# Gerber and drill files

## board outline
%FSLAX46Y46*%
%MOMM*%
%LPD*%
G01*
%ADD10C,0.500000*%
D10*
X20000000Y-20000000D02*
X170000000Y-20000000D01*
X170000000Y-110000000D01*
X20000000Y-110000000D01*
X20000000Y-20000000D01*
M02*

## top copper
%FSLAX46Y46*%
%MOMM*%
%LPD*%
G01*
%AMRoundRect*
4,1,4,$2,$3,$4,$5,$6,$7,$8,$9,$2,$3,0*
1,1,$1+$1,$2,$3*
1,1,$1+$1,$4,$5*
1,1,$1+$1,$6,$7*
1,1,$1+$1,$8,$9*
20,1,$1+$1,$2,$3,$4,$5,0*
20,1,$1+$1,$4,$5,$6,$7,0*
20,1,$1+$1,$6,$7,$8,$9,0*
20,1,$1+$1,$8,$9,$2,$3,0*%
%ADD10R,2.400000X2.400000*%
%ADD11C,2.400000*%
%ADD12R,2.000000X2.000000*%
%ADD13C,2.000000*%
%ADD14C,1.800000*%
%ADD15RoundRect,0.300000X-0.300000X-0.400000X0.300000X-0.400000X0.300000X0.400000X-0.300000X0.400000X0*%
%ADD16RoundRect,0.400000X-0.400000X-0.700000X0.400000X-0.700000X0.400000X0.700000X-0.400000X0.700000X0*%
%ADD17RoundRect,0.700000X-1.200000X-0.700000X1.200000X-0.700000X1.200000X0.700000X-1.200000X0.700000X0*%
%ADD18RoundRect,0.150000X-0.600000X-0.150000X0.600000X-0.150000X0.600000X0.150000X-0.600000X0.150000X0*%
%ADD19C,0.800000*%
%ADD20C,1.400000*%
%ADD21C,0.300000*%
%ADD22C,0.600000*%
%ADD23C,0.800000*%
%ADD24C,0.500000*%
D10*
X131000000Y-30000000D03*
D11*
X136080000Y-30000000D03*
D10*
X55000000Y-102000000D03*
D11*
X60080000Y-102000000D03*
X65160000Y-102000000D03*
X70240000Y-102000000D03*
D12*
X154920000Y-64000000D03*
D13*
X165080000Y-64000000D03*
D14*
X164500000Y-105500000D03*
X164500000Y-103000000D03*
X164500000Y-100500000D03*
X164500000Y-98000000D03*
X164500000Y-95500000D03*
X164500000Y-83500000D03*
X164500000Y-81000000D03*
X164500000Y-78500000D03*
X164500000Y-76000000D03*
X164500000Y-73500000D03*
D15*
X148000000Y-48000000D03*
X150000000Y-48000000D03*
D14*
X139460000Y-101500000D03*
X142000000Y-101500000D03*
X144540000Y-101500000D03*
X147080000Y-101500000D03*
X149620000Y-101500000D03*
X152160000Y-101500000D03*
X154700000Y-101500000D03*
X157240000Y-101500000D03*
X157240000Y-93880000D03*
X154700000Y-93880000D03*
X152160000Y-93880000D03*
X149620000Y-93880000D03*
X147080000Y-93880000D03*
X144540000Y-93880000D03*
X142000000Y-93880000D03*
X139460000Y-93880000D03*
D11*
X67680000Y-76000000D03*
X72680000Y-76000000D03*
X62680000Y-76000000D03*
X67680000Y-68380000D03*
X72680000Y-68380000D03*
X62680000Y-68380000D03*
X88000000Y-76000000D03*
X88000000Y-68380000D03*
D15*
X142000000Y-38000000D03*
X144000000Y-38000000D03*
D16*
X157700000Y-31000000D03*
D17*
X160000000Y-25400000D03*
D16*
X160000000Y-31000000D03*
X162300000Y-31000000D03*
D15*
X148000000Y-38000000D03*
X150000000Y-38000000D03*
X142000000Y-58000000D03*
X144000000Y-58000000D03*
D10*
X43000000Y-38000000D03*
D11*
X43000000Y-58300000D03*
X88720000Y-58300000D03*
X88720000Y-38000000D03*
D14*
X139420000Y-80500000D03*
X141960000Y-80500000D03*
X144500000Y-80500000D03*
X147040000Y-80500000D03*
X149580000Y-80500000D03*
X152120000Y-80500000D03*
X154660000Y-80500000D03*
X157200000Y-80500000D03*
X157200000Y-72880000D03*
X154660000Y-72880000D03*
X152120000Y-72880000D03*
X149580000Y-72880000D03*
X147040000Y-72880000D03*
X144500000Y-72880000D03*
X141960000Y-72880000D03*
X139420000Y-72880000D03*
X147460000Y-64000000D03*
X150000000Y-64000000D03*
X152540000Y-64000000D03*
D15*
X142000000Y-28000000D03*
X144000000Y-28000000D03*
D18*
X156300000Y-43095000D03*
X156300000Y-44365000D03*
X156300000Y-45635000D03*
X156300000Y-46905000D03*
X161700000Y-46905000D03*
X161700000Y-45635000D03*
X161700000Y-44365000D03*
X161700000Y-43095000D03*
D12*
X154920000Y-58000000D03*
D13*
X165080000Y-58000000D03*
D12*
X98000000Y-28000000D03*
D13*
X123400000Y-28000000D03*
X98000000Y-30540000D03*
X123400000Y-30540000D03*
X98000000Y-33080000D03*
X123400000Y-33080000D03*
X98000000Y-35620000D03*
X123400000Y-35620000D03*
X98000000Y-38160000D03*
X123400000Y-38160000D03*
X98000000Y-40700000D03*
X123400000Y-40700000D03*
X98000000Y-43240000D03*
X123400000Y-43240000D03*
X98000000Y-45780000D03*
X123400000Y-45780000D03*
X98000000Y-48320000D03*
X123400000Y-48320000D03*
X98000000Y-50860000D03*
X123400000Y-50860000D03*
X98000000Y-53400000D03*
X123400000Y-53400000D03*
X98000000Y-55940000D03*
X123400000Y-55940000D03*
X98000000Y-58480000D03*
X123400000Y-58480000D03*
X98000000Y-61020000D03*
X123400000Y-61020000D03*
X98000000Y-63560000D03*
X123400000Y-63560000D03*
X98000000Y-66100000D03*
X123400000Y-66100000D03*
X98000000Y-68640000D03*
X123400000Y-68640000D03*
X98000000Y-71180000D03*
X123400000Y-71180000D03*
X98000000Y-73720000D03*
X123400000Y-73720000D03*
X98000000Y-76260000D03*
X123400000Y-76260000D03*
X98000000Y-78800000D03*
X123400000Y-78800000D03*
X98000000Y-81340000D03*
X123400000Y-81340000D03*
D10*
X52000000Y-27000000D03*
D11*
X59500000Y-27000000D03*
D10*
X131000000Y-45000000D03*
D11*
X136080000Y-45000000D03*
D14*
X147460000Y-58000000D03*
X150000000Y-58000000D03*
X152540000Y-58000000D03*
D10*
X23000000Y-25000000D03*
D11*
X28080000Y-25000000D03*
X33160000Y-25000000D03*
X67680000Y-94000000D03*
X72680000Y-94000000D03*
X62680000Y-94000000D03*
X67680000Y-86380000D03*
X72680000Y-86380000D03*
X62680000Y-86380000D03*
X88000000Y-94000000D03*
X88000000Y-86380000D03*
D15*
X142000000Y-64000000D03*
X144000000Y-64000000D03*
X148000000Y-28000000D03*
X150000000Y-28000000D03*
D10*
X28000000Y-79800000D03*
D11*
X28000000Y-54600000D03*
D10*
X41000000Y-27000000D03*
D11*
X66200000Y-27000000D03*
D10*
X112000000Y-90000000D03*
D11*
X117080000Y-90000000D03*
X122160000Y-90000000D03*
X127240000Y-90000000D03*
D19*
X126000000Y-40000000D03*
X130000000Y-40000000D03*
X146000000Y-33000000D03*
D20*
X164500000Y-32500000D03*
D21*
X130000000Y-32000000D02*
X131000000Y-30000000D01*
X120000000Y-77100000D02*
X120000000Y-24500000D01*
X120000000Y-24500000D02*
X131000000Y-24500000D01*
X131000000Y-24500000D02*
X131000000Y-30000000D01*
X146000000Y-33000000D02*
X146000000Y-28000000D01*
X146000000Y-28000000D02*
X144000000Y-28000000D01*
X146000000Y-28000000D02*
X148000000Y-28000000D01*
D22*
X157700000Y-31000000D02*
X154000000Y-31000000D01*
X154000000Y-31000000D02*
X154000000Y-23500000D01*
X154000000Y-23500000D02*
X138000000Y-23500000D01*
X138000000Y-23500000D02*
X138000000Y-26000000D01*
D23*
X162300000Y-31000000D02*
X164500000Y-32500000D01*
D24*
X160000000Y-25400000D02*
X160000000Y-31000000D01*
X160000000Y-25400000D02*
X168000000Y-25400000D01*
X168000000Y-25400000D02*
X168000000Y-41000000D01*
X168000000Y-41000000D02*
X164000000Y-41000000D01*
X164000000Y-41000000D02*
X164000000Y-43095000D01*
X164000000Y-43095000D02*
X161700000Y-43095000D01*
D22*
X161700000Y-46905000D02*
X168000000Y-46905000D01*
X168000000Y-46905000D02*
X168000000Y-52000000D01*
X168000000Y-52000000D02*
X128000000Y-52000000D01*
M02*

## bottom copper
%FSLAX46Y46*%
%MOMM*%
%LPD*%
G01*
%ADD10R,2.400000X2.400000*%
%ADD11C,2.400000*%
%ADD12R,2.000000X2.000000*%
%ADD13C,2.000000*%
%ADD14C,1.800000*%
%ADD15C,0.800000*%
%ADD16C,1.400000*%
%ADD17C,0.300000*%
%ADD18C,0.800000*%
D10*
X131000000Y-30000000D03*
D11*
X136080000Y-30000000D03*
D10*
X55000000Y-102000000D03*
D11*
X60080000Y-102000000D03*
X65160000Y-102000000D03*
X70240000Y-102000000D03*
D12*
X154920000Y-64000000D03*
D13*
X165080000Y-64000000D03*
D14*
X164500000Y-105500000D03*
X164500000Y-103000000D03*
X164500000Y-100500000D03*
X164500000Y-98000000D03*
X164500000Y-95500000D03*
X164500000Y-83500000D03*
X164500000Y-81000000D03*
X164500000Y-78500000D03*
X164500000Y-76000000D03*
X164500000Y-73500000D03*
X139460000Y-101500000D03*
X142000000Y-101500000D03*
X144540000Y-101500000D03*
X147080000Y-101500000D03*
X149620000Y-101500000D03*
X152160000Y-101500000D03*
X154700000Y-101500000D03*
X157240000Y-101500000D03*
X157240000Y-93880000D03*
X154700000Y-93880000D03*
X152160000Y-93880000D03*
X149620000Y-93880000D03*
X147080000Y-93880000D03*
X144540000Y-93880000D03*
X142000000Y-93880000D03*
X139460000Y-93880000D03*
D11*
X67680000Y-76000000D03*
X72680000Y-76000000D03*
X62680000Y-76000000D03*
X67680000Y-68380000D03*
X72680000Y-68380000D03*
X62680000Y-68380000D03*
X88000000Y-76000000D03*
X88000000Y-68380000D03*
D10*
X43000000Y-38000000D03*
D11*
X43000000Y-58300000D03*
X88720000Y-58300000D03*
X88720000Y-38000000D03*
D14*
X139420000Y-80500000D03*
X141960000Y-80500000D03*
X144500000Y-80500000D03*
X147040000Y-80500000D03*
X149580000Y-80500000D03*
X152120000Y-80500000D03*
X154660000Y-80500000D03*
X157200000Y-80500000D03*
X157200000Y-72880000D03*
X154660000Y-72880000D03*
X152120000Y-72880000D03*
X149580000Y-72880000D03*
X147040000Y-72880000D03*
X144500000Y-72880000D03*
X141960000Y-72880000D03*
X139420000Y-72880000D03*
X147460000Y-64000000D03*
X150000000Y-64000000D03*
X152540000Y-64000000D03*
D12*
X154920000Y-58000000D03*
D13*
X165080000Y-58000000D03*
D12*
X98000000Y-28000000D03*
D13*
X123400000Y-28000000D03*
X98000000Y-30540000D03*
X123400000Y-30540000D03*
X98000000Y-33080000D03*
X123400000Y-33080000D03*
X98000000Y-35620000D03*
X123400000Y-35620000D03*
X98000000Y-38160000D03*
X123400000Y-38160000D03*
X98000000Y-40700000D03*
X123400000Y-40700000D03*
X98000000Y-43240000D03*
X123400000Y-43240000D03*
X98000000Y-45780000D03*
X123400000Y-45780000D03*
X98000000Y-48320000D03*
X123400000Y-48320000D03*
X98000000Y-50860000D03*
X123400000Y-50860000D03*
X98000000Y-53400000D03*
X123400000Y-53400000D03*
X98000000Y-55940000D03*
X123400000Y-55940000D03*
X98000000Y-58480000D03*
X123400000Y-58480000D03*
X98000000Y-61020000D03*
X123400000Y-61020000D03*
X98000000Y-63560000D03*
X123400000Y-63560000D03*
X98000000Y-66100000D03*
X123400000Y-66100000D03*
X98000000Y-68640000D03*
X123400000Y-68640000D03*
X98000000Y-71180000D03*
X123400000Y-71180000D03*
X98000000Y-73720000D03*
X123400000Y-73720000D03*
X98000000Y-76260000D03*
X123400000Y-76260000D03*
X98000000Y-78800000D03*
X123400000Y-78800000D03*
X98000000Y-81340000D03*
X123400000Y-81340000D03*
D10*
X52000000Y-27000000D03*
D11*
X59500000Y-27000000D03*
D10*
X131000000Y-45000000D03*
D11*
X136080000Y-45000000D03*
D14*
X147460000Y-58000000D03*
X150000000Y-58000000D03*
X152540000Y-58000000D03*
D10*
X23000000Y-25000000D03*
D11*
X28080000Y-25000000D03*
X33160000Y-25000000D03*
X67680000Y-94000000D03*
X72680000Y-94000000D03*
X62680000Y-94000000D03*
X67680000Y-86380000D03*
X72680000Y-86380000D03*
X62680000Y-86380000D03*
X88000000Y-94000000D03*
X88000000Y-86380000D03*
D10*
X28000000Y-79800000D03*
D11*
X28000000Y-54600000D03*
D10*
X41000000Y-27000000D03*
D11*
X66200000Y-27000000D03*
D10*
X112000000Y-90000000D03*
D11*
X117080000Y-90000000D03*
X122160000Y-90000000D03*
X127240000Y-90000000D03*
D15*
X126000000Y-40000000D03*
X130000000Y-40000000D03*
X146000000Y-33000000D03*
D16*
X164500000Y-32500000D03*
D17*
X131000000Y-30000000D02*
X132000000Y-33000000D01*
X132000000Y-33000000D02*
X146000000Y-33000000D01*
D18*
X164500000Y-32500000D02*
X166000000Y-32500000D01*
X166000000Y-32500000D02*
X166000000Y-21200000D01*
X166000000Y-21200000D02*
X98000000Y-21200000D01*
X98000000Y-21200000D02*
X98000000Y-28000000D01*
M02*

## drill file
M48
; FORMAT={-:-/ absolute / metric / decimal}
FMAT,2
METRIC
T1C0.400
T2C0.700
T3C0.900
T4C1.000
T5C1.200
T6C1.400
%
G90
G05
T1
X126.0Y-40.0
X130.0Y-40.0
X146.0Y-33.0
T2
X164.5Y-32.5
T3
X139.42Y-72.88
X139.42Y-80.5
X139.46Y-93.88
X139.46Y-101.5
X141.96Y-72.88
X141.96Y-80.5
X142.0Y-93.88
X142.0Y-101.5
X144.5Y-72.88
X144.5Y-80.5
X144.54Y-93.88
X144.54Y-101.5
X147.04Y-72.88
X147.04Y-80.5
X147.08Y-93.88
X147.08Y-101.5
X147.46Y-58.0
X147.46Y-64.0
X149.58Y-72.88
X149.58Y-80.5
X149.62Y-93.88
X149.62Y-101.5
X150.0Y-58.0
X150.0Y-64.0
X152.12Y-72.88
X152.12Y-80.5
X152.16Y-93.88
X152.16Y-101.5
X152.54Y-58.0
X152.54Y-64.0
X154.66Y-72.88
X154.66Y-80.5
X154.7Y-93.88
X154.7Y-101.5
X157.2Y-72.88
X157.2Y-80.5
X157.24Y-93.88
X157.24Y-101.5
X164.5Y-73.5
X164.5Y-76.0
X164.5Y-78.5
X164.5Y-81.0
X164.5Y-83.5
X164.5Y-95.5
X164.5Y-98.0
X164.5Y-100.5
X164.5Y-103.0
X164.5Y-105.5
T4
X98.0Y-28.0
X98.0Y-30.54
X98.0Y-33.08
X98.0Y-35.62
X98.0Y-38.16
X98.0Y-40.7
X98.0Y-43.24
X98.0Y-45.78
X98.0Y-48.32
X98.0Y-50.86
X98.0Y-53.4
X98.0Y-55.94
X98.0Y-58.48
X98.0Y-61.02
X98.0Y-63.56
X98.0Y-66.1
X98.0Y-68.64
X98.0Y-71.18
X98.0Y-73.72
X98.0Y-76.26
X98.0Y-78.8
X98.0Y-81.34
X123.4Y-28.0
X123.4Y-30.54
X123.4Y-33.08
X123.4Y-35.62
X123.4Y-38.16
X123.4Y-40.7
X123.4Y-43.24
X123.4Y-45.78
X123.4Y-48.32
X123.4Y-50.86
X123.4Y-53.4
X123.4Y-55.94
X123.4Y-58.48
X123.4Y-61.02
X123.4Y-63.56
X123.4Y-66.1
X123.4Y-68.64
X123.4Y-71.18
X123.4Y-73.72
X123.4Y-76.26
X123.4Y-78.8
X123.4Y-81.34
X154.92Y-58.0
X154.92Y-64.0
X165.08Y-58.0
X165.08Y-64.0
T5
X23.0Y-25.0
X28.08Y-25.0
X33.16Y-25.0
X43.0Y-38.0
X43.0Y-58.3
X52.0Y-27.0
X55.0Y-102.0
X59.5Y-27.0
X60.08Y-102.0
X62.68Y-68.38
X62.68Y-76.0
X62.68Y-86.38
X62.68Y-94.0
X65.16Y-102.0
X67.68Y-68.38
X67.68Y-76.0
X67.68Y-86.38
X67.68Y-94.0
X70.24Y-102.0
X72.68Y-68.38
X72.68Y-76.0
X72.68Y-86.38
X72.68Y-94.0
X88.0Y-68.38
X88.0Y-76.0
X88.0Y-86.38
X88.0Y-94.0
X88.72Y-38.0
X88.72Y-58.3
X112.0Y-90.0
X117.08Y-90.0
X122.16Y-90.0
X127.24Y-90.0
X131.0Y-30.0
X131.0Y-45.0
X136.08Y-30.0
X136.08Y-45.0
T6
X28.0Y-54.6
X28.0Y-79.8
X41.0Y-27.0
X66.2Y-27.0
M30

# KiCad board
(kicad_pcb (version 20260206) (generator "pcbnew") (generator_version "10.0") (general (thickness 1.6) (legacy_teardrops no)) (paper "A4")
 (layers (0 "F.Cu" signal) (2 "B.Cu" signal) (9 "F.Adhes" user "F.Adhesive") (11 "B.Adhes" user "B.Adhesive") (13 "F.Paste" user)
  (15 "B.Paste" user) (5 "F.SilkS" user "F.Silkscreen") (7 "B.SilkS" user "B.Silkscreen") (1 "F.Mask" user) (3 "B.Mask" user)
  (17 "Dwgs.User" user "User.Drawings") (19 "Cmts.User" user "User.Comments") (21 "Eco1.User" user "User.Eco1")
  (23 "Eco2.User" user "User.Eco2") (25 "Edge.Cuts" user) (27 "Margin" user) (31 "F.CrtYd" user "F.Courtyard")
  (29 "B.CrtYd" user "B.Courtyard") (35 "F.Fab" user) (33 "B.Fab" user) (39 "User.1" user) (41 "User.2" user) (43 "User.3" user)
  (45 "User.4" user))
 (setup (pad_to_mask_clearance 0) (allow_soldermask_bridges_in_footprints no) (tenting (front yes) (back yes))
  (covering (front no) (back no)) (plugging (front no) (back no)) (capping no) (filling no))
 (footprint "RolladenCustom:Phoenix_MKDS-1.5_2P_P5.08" (layer "F.Cu") (at 131 30)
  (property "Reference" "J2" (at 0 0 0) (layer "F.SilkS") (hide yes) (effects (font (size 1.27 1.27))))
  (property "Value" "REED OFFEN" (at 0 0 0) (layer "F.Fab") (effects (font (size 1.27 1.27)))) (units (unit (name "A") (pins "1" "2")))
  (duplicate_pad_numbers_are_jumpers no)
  (pad "1" thru_hole rect (at 0 0) (size 2.4 2.4) (drill 1.2) (layers "*.Cu" "*.Mask") (remove_unused_layers no) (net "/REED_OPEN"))
  (pad "2" thru_hole circle (at 5.08 0) (size 2.4 2.4) (drill 1.2) (layers "*.Cu" "*.Mask") (remove_unused_layers no) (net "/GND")))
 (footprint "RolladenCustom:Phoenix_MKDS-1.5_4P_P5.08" (layer "F.Cu") (at 55 102)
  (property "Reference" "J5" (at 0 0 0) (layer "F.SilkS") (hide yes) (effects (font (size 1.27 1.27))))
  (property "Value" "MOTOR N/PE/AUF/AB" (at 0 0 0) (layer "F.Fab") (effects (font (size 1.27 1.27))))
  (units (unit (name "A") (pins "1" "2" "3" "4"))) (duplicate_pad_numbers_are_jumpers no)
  (pad "1" thru_hole rect (at 0 0) (size 2.4 2.4) (drill 1.2) (layers "*.Cu" "*.Mask") (remove_unused_layers no) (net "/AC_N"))
  (pad "2" thru_hole circle (at 5.08 0) (size 2.4 2.4) (drill 1.2) (layers "*.Cu" "*.Mask") (remove_unused_layers no) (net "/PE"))
  (pad "3" thru_hole circle (at 10.16 0) (size 2.4 2.4) (drill 1.2) (layers "*.Cu" "*.Mask") (remove_unused_layers no) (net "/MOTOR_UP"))
  (pad "4" thru_hole circle (at 15.24 0) (size 2.4 2.4) (drill 1.2) (layers "*.Cu" "*.Mask") (remove_unused_layers no) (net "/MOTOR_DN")))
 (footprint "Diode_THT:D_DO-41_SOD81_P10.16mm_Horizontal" (layer "F.Cu") (at 160 64)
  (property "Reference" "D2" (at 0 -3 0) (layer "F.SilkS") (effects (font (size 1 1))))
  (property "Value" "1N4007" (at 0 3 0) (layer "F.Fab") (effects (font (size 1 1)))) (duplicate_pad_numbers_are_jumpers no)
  (pad "1" thru_hole rect (at -5.08 0) (size 2 2) (drill 1) (layers "*.Cu" "*.Mask") (remove_unused_layers no) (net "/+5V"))
  (pad "2" thru_hole circle (at 5.08 0) (size 2 2) (drill 1) (layers "*.Cu" "*.Mask") (remove_unused_layers no) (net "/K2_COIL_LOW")))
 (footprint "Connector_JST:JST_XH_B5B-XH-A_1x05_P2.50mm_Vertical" (layer "F.Cu") (at 164.5 105.5 90)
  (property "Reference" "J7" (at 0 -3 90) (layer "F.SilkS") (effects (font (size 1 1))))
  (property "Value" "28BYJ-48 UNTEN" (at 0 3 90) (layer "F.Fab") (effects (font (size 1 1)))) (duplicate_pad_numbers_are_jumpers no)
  (pad "1" thru_hole circle (at 0 0 90) (size 1.8 1.8) (drill 0.9) (layers "*.Cu" "*.Mask") (remove_unused_layers no) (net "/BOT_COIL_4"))
  (pad "2" thru_hole circle (at 2.5 0 90) (size 1.8 1.8) (drill 0.9) (layers "*.Cu" "*.Mask") (remove_unused_layers no) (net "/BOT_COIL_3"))
  (pad "3" thru_hole circle (at 5 0 90) (size 1.8 1.8) (drill 0.9) (layers "*.Cu" "*.Mask") (remove_unused_layers no) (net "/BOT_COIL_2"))
  (pad "4" thru_hole circle (at 7.5 0 90) (size 1.8 1.8) (drill 0.9) (layers "*.Cu" "*.Mask") (remove_unused_layers no) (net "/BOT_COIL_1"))
  (pad "5" thru_hole circle (at 10 0 90) (size 1.8 1.8) (drill 0.9) (layers "*.Cu" "*.Mask") (remove_unused_layers no) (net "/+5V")))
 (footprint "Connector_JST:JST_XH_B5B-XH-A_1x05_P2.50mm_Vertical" (layer "F.Cu") (at 164.5 83.5 90)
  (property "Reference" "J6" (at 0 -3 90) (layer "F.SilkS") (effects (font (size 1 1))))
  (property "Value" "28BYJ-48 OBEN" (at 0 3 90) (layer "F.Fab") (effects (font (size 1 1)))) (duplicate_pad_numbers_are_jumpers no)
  (pad "1" thru_hole circle (at 0 0 90) (size 1.8 1.8) (drill 0.9) (layers "*.Cu" "*.Mask") (remove_unused_layers no) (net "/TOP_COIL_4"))
  (pad "2" thru_hole circle (at 2.5 0 90) (size 1.8 1.8) (drill 0.9) (layers "*.Cu" "*.Mask") (remove_unused_layers no) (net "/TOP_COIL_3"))
  (pad "3" thru_hole circle (at 5 0 90) (size 1.8 1.8) (drill 0.9) (layers "*.Cu" "*.Mask") (remove_unused_layers no) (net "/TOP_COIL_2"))
  (pad "4" thru_hole circle (at 7.5 0 90) (size 1.8 1.8) (drill 0.9) (layers "*.Cu" "*.Mask") (remove_unused_layers no) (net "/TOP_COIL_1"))
  (pad "5" thru_hole circle (at 10 0 90) (size 1.8 1.8) (drill 0.9) (layers "*.Cu" "*.Mask") (remove_unused_layers no) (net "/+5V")))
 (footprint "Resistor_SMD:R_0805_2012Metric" (layer "F.Cu") (at 149 48)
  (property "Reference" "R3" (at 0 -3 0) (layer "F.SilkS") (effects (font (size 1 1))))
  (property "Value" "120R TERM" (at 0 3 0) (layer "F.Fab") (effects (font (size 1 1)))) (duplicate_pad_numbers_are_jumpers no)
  (pad "1" smd roundrect (at -1 0) (size 1.2 1.4) (layers "F.Cu" "F.Mask" "F.Paste") (roundrect_rratio 0.25) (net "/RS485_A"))
  (pad "2" smd roundrect (at 1 0) (size 1.2 1.4) (layers "F.Cu" "F.Mask" "F.Paste") (roundrect_rratio 0.25) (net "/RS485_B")))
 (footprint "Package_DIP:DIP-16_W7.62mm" (layer "F.Cu") (at 139.46 101.5 90)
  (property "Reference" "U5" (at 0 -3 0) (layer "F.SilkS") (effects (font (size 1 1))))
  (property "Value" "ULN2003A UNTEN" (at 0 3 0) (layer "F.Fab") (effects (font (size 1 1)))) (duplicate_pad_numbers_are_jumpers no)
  (pad "1" thru_hole circle (at 0 0) (size 1.8 1.8) (drill 0.9) (layers "*.Cu" "*.Mask") (remove_unused_layers no) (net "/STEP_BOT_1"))
  (pad "2" thru_hole circle (at 0 2.54) (size 1.8 1.8) (drill 0.9) (layers "*.Cu" "*.Mask") (remove_unused_layers no) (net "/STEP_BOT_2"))
  (pad "3" thru_hole circle (at 0 5.08) (size 1.8 1.8) (drill 0.9) (layers "*.Cu" "*.Mask") (remove_unused_layers no) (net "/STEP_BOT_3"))
  (pad "4" thru_hole circle (at 0 7.62) (size 1.8 1.8) (drill 0.9) (layers "*.Cu" "*.Mask") (remove_unused_layers no) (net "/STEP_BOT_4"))
  (pad "5" thru_hole circle (at 0 10.16) (size 1.8 1.8) (drill 0.9) (layers "*.Cu" "*.Mask") (remove_unused_layers no))
  (pad "6" thru_hole circle (at 0 12.7) (size 1.8 1.8) (drill 0.9) (layers "*.Cu" "*.Mask") (remove_unused_layers no))
  (pad "7" thru_hole circle (at 0 15.24) (size 1.8 1.8) (drill 0.9) (layers "*.Cu" "*.Mask") (remove_unused_layers no))
  (pad "8" thru_hole circle (at 0 17.78) (size 1.8 1.8) (drill 0.9) (layers "*.Cu" "*.Mask") (remove_unused_layers no) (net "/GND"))
  (pad "9" thru_hole circle (at 7.62 17.78) (size 1.8 1.8) (drill 0.9) (layers "*.Cu" "*.Mask") (remove_unused_layers no) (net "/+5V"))
  (pad "10" thru_hole circle (at 7.62 15.24) (size 1.8 1.8) (drill 0.9) (layers "*.Cu" "*.Mask") (remove_unused_layers no))
  (pad "11" thru_hole circle (at 7.62 12.7) (size 1.8 1.8) (drill 0.9) (layers "*.Cu" "*.Mask") (remove_unused_layers no))
  (pad "12" thru_hole circle (at 7.62 10.16) (size 1.8 1.8) (drill 0.9) (layers "*.Cu" "*.Mask") (remove_unused_layers no))
  (pad "13" thru_hole circle (at 7.62 7.62) (size 1.8 1.8) (drill 0.9) (layers "*.Cu" "*.Mask") (remove_unused_layers no)
   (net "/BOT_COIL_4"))
  (pad "14" thru_hole circle (at 7.62 5.08) (size 1.8 1.8) (drill 0.9) (layers "*.Cu" "*.Mask") (remove_unused_layers no)
   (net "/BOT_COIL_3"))
  (pad "15" thru_hole circle (at 7.62 2.54) (size 1.8 1.8) (drill 0.9) (layers "*.Cu" "*.Mask") (remove_unused_layers no)
   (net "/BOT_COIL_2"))
  (pad "16" thru_hole circle (at 7.62 0) (size 1.8 1.8) (drill 0.9) (layers "*.Cu" "*.Mask") (remove_unused_layers no) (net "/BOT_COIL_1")))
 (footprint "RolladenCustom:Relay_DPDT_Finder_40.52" (layer "F.Cu") (at 88 76 180)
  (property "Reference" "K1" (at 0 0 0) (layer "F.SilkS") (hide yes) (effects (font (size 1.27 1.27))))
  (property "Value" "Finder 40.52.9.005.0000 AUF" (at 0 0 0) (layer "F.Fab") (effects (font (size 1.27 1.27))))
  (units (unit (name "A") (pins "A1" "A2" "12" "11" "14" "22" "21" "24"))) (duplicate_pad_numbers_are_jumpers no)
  (pad "11" thru_hole circle (at 20.32 0) (size 2.4 2.4) (drill 1.2) (layers "*.Cu" "*.Mask") (remove_unused_layers no) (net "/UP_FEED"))
  (pad "12" thru_hole circle (at 15.32 0) (size 2.4 2.4) (drill 1.2) (layers "*.Cu" "*.Mask") (remove_unused_layers no)
   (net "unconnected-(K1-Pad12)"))
  (pad "14" thru_hole circle (at 25.32 0) (size 2.4 2.4) (drill 1.2) (layers "*.Cu" "*.Mask") (remove_unused_layers no) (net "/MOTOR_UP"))
  (pad "21" thru_hole circle (at 20.32 7.62) (size 2.4 2.4) (drill 1.2) (layers "*.Cu" "*.Mask") (remove_unused_layers no) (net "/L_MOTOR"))
  (pad "22" thru_hole circle (at 15.32 7.62) (size 2.4 2.4) (drill 1.2) (layers "*.Cu" "*.Mask") (remove_unused_layers no) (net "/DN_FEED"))
  (pad "24" thru_hole circle (at 25.32 7.62) (size 2.4 2.4) (drill 1.2) (layers "*.Cu" "*.Mask") (remove_unused_layers no)
   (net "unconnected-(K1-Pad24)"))
  (pad "A1" thru_hole circle (at 0 0) (size 2.4 2.4) (drill 1.2) (layers "*.Cu" "*.Mask") (remove_unused_layers no) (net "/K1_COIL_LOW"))
  (pad "A2" thru_hole circle (at 0 7.62) (size 2.4 2.4) (drill 1.2) (layers "*.Cu" "*.Mask") (remove_unused_layers no) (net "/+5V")))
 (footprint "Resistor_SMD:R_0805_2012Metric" (layer "F.Cu") (at 143 38)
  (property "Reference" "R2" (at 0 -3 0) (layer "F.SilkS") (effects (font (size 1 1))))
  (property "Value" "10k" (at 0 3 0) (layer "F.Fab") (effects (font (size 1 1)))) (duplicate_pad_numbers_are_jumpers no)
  (pad "1" smd roundrect (at -1 0) (size 1.2 1.4) (layers "F.Cu" "F.Mask" "F.Paste") (roundrect_rratio 0.25) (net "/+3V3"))
  (pad "2" smd roundrect (at 1 0) (size 1.2 1.4) (layers "F.Cu" "F.Mask" "F.Paste") (roundrect_rratio 0.25) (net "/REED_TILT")))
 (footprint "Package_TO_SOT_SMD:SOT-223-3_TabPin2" (layer "F.Cu") (at 160 28)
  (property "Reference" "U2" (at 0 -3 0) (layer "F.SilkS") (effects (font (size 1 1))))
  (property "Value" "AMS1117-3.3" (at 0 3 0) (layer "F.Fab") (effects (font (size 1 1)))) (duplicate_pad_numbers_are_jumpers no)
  (pad "1" smd roundrect (at -2.3 3) (size 1.6 2.2) (layers "F.Cu" "F.Mask" "F.Paste") (roundrect_rratio 0.25) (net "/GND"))
  (pad "2" smd roundrect (at 0 -2.6) (size 3.8 2.8) (layers "F.Cu" "F.Mask" "F.Paste") (roundrect_rratio 0.25) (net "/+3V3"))
  (pad "2" smd roundrect (at 0 3) (size 1.6 2.2) (layers "F.Cu" "F.Mask" "F.Paste") (roundrect_rratio 0.25) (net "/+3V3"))
  (pad "3" smd roundrect (at 2.3 3) (size 1.6 2.2) (layers "F.Cu" "F.Mask" "F.Paste") (roundrect_rratio 0.25) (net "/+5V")))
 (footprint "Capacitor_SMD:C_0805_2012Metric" (layer "F.Cu") (at 149 38)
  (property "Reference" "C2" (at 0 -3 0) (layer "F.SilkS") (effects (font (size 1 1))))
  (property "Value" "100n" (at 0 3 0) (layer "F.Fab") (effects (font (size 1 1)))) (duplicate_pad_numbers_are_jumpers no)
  (pad "1" smd roundrect (at -1 0) (size 1.2 1.4) (layers "F.Cu" "F.Mask" "F.Paste") (roundrect_rratio 0.25) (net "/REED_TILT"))
  (pad "2" smd roundrect (at 1 0) (size 1.2 1.4) (layers "F.Cu" "F.Mask" "F.Paste") (roundrect_rratio 0.25) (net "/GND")))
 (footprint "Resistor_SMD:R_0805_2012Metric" (layer "F.Cu") (at 143 58)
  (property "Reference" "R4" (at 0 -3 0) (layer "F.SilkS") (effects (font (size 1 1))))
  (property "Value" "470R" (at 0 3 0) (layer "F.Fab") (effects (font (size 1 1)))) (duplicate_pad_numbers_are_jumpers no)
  (pad "1" smd roundrect (at -1 0) (size 1.2 1.4) (layers "F.Cu" "F.Mask" "F.Paste") (roundrect_rratio 0.25) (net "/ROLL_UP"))
  (pad "2" smd roundrect (at 1 0) (size 1.2 1.4) (layers "F.Cu" "F.Mask" "F.Paste") (roundrect_rratio 0.25) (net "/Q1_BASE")))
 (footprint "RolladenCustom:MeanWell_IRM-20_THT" (layer "F.Cu") (at 43 38)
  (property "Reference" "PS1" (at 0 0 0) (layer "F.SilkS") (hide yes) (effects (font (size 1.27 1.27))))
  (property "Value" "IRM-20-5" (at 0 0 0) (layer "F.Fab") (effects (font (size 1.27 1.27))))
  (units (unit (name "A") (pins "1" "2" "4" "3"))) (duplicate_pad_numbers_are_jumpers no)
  (pad "1" thru_hole rect (at 0 0) (size 2.4 2.4) (drill 1.2) (layers "*.Cu" "*.Mask") (remove_unused_layers no) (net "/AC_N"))
  (pad "2" thru_hole circle (at 0 20.3) (size 2.4 2.4) (drill 1.2) (layers "*.Cu" "*.Mask") (remove_unused_layers no) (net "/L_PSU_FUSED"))
  (pad "3" thru_hole circle (at 45.72 20.3) (size 2.4 2.4) (drill 1.2) (layers "*.Cu" "*.Mask") (remove_unused_layers no) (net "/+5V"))
  (pad "4" thru_hole circle (at 45.72 0) (size 2.4 2.4) (drill 1.2) (layers "*.Cu" "*.Mask") (remove_unused_layers no) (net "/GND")))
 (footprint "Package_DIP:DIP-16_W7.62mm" (layer "F.Cu") (at 139.42 80.5 90)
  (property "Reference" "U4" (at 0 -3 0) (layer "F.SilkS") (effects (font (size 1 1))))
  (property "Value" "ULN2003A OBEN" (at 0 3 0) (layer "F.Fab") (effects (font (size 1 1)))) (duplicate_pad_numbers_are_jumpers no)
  (pad "1" thru_hole circle (at 0 0) (size 1.8 1.8) (drill 0.9) (layers "*.Cu" "*.Mask") (remove_unused_layers no) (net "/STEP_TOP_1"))
  (pad "2" thru_hole circle (at 0 2.54) (size 1.8 1.8) (drill 0.9) (layers "*.Cu" "*.Mask") (remove_unused_layers no) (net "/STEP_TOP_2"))
  (pad "3" thru_hole circle (at 0 5.08) (size 1.8 1.8) (drill 0.9) (layers "*.Cu" "*.Mask") (remove_unused_layers no) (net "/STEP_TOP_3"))
  (pad "4" thru_hole circle (at 0 7.62) (size 1.8 1.8) (drill 0.9) (layers "*.Cu" "*.Mask") (remove_unused_layers no) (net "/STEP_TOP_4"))
  (pad "5" thru_hole circle (at 0 10.16) (size 1.8 1.8) (drill 0.9) (layers "*.Cu" "*.Mask") (remove_unused_layers no))
  (pad "6" thru_hole circle (at 0 12.7) (size 1.8 1.8) (drill 0.9) (layers "*.Cu" "*.Mask") (remove_unused_layers no))
  (pad "7" thru_hole circle (at 0 15.24) (size 1.8 1.8) (drill 0.9) (layers "*.Cu" "*.Mask") (remove_unused_layers no))
  (pad "8" thru_hole circle (at 0 17.78) (size 1.8 1.8) (drill 0.9) (layers "*.Cu" "*.Mask") (remove_unused_layers no) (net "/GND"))
  (pad "9" thru_hole circle (at 7.62 17.78) (size 1.8 1.8) (drill 0.9) (layers "*.Cu" "*.Mask") (remove_unused_layers no) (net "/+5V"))
  (pad "10" thru_hole circle (at 7.62 15.24) (size 1.8 1.8) (drill 0.9) (layers "*.Cu" "*.Mask") (remove_unused_layers no))
  (pad "11" thru_hole circle (at 7.62 12.7) (size 1.8 1.8) (drill 0.9) (layers "*.Cu" "*.Mask") (remove_unused_layers no))
  (pad "12" thru_hole circle (at 7.62 10.16) (size 1.8 1.8) (drill 0.9) (layers "*.Cu" "*.Mask") (remove_unused_layers no))
  (pad "13" thru_hole circle (at 7.62 7.62) (size 1.8 1.8) (drill 0.9) (layers "*.Cu" "*.Mask") (remove_unused_layers no)
   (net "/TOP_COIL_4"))
  (pad "14" thru_hole circle (at 7.62 5.08) (size 1.8 1.8) (drill 0.9) (layers "*.Cu" "*.Mask") (remove_unused_layers no)
   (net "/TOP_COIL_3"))
  (pad "15" thru_hole circle (at 7.62 2.54) (size 1.8 1.8) (drill 0.9) (layers "*.Cu" "*.Mask") (remove_unused_layers no)
   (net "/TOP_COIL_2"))
  (pad "16" thru_hole circle (at 7.62 0) (size 1.8 1.8) (drill 0.9) (layers "*.Cu" "*.Mask") (remove_unused_layers no) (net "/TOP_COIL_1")))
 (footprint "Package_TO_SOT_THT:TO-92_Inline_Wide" (layer "F.Cu") (at 150 64)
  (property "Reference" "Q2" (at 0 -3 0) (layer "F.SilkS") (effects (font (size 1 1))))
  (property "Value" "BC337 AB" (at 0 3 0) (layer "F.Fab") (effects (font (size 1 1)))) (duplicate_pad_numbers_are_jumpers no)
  (pad "1" thru_hole circle (at -2.54 0) (size 1.8 1.8) (drill 0.9) (layers "*.Cu" "*.Mask") (remove_unused_layers no) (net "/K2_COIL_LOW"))
  (pad "2" thru_hole circle (at 0 0) (size 1.8 1.8) (drill 0.9) (layers "*.Cu" "*.Mask") (remove_unused_layers no) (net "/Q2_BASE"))
  (pad "3" thru_hole circle (at 2.54 0) (size 1.8 1.8) (drill 0.9) (layers "*.Cu" "*.Mask") (remove_unused_layers no) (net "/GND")))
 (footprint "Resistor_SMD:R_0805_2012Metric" (layer "F.Cu") (at 143 28)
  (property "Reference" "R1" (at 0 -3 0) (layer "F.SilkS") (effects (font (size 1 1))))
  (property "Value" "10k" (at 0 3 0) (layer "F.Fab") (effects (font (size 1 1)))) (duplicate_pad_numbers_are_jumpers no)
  (pad "1" smd roundrect (at -1 0) (size 1.2 1.4) (layers "F.Cu" "F.Mask" "F.Paste") (roundrect_rratio 0.25) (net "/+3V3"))
  (pad "2" smd roundrect (at 1 0) (size 1.2 1.4) (layers "F.Cu" "F.Mask" "F.Paste") (roundrect_rratio 0.25) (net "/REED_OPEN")))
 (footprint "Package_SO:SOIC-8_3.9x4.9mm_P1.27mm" (layer "F.Cu") (at 159 45)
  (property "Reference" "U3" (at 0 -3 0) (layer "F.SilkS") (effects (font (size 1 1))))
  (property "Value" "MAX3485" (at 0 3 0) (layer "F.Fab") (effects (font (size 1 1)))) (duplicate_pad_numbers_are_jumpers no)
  (pad "1" smd roundrect (at -2.7 -1.905) (size 1.5 0.6) (layers "F.Cu" "F.Mask" "F.Paste") (roundrect_rratio 0.25) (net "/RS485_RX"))
  (pad "2" smd roundrect (at -2.7 -0.635) (size 1.5 0.6) (layers "F.Cu" "F.Mask" "F.Paste") (roundrect_rratio 0.25) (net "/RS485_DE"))
  (pad "3" smd roundrect (at -2.7 0.635) (size 1.5 0.6) (layers "F.Cu" "F.Mask" "F.Paste") (roundrect_rratio 0.25) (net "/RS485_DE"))
  (pad "4" smd roundrect (at -2.7 1.905) (size 1.5 0.6) (layers "F.Cu" "F.Mask" "F.Paste") (roundrect_rratio 0.25) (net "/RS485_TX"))
  (pad "5" smd roundrect (at 2.7 1.905) (size 1.5 0.6) (layers "F.Cu" "F.Mask" "F.Paste") (roundrect_rratio 0.25) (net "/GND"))
  (pad "6" smd roundrect (at 2.7 0.635) (size 1.5 0.6) (layers "F.Cu" "F.Mask" "F.Paste") (roundrect_rratio 0.25) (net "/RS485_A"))
  (pad "7" smd roundrect (at 2.7 -0.635) (size 1.5 0.6) (layers "F.Cu" "F.Mask" "F.Paste") (roundrect_rratio 0.25) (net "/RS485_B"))
  (pad "8" smd roundrect (at 2.7 -1.905) (size 1.5 0.6) (layers "F.Cu" "F.Mask" "F.Paste") (roundrect_rratio 0.25) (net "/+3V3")))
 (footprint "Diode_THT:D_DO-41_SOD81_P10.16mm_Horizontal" (layer "F.Cu") (at 160 58)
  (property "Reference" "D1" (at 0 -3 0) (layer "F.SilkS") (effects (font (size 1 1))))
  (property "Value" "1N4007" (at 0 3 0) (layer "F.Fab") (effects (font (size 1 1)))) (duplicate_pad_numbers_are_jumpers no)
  (pad "1" thru_hole rect (at -5.08 0) (size 2 2) (drill 1) (layers "*.Cu" "*.Mask") (remove_unused_layers no) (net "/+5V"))
  (pad "2" thru_hole circle (at 5.08 0) (size 2 2) (drill 1) (layers "*.Cu" "*.Mask") (remove_unused_layers no) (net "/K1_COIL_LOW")))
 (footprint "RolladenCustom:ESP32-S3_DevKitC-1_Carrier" (layer "F.Cu") (at 98 28)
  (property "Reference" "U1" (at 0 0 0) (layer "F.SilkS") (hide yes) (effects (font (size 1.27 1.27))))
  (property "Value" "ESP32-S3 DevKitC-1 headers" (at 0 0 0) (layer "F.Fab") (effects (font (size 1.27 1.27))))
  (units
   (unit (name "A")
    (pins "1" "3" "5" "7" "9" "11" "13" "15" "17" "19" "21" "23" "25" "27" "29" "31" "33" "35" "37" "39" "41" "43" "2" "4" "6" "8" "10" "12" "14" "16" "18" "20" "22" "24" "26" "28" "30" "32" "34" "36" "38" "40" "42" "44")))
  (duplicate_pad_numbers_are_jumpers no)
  (pad "1" thru_hole rect (at 0 0) (size 2 2) (drill 1) (layers "*.Cu" "*.Mask") (remove_unused_layers no) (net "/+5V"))
  (pad "2" thru_hole circle (at 25.4 0) (size 2 2) (drill 1) (layers "*.Cu" "*.Mask") (remove_unused_layers no) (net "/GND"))
  (pad "3" thru_hole circle (at 0 2.54) (size 2 2) (drill 1) (layers "*.Cu" "*.Mask") (remove_unused_layers no) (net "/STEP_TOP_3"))
  (pad "4" thru_hole circle (at 25.4 2.54) (size 2 2) (drill 1) (layers "*.Cu" "*.Mask") (remove_unused_layers no)
   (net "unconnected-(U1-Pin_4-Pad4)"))
  (pad "5" thru_hole circle (at 0 5.08) (size 2 2) (drill 1) (layers "*.Cu" "*.Mask") (remove_unused_layers no) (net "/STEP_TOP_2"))
  (pad "6" thru_hole circle (at 25.4 5.08) (size 2 2) (drill 1) (layers "*.Cu" "*.Mask") (remove_unused_layers no)
   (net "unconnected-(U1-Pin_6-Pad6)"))
  (pad "7" thru_hole circle (at 0 7.62) (size 2 2) (drill 1) (layers "*.Cu" "*.Mask") (remove_unused_layers no) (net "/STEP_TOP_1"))
  (pad "8" thru_hole circle (at 25.4 7.62) (size 2 2) (drill 1) (layers "*.Cu" "*.Mask") (remove_unused_layers no)
   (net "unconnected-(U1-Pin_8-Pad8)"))
  (pad "9" thru_hole circle (at 0 10.16) (size 2 2) (drill 1) (layers "*.Cu" "*.Mask") (remove_unused_layers no) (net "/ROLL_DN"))
  (pad "10" thru_hole circle (at 25.4 10.16) (size 2 2) (drill 1) (layers "*.Cu" "*.Mask") (remove_unused_layers no)
   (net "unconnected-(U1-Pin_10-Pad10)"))
  (pad "11" thru_hole circle (at 0 12.7) (size 2 2) (drill 1) (layers "*.Cu" "*.Mask") (remove_unused_layers no) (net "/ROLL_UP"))
  (pad "12" thru_hole circle (at 25.4 12.7) (size 2 2) (drill 1) (layers "*.Cu" "*.Mask") (remove_unused_layers no)
   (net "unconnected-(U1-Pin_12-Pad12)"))
  (pad "13" thru_hole circle (at 0 15.24) (size 2 2) (drill 1) (layers "*.Cu" "*.Mask") (remove_unused_layers no)
   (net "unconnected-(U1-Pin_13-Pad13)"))
  (pad "14" thru_hole circle (at 25.4 15.24) (size 2 2) (drill 1) (layers "*.Cu" "*.Mask") (remove_unused_layers no)
   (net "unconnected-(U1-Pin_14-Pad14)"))
  (pad "15" thru_hole circle (at 0 17.78) (size 2 2) (drill 1) (layers "*.Cu" "*.Mask") (remove_unused_layers no)
   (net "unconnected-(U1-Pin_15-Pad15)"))
  (pad "16" thru_hole circle (at 25.4 17.78) (size 2 2) (drill 1) (layers "*.Cu" "*.Mask") (remove_unused_layers no)
   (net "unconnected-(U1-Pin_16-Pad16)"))
  (pad "17" thru_hole circle (at 0 20.32) (size 2 2) (drill 1) (layers "*.Cu" "*.Mask") (remove_unused_layers no)
   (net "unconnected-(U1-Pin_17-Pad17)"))
  (pad "18" thru_hole circle (at 25.4 20.32) (size 2 2) (drill 1) (layers "*.Cu" "*.Mask") (remove_unused_layers no)
   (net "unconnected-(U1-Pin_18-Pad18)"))
  (pad "19" thru_hole circle (at 0 22.86) (size 2 2) (drill 1) (layers "*.Cu" "*.Mask") (remove_unused_layers no)
   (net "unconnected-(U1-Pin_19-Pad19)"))
  (pad "20" thru_hole circle (at 25.4 22.86) (size 2 2) (drill 1) (layers "*.Cu" "*.Mask") (remove_unused_layers no)
   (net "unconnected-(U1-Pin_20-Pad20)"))
  (pad "21" thru_hole circle (at 0 25.4) (size 2 2) (drill 1) (layers "*.Cu" "*.Mask") (remove_unused_layers no) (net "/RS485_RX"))
  (pad "22" thru_hole circle (at 25.4 25.4) (size 2 2) (drill 1) (layers "*.Cu" "*.Mask") (remove_unused_layers no)
   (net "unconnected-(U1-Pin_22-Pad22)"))
  (pad "23" thru_hole circle (at 0 27.94) (size 2 2) (drill 1) (layers "*.Cu" "*.Mask") (remove_unused_layers no) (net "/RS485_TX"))
  (pad "24" thru_hole circle (at 25.4 27.94) (size 2 2) (drill 1) (layers "*.Cu" "*.Mask") (remove_unused_layers no) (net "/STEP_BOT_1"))
  (pad "25" thru_hole circle (at 0 30.48) (size 2 2) (drill 1) (layers "*.Cu" "*.Mask") (remove_unused_layers no) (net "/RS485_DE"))
  (pad "26" thru_hole circle (at 25.4 30.48) (size 2 2) (drill 1) (layers "*.Cu" "*.Mask") (remove_unused_layers no) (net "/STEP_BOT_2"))
  (pad "27" thru_hole circle (at 0 33.02) (size 2 2) (drill 1) (layers "*.Cu" "*.Mask") (remove_unused_layers no) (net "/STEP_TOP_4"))
  (pad "28" thru_hole circle (at 25.4 33.02) (size 2 2) (drill 1) (layers "*.Cu" "*.Mask") (remove_unused_layers no) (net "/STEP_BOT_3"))
  (pad "29" thru_hole circle (at 0 35.56) (size 2 2) (drill 1) (layers "*.Cu" "*.Mask") (remove_unused_layers no)
   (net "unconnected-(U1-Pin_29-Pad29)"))
  (pad "30" thru_hole circle (at 25.4 35.56) (size 2 2) (drill 1) (layers "*.Cu" "*.Mask") (remove_unused_layers no) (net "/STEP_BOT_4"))
  (pad "31" thru_hole circle (at 0 38.1) (size 2 2) (drill 1) (layers "*.Cu" "*.Mask") (remove_unused_layers no)
   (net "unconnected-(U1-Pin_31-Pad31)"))
  (pad "32" thru_hole circle (at 25.4 38.1) (size 2 2) (drill 1) (layers "*.Cu" "*.Mask") (remove_unused_layers no)
   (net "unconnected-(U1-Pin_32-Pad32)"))
  (pad "33" thru_hole circle (at 0 40.64) (size 2 2) (drill 1) (layers "*.Cu" "*.Mask") (remove_unused_layers no) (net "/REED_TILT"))
  (pad "34" thru_hole circle (at 25.4 40.64) (size 2 2) (drill 1) (layers "*.Cu" "*.Mask") (remove_unused_layers no)
   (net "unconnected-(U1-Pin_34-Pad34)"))
  (pad "35" thru_hole circle (at 0 43.18) (size 2 2) (drill 1) (layers "*.Cu" "*.Mask") (remove_unused_layers no) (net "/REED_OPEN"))
  (pad "36" thru_hole circle (at 25.4 43.18) (size 2 2) (drill 1) (layers "*.Cu" "*.Mask") (remove_unused_layers no)
   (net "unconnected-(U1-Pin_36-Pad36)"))
  (pad "37" thru_hole circle (at 0 45.72) (size 2 2) (drill 1) (layers "*.Cu" "*.Mask") (remove_unused_layers no)
   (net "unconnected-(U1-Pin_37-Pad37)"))
  (pad "38" thru_hole circle (at 25.4 45.72) (size 2 2) (drill 1) (layers "*.Cu" "*.Mask") (remove_unused_layers no)
   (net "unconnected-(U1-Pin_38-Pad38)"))
  (pad "39" thru_hole circle (at 0 48.26) (size 2 2) (drill 1) (layers "*.Cu" "*.Mask") (remove_unused_layers no)
   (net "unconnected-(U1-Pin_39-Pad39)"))
  (pad "40" thru_hole circle (at 25.4 48.26) (size 2 2) (drill 1) (layers "*.Cu" "*.Mask") (remove_unused_layers no)
   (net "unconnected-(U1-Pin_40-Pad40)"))
  (pad "41" thru_hole circle (at 0 50.8) (size 2 2) (drill 1) (layers "*.Cu" "*.Mask") (remove_unused_layers no)
   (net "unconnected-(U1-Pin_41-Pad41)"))
  (pad "42" thru_hole circle (at 25.4 50.8) (size 2 2) (drill 1) (layers "*.Cu" "*.Mask") (remove_unused_layers no) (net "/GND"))
  (pad "43" thru_hole circle (at 0 53.34) (size 2 2) (drill 1) (layers "*.Cu" "*.Mask") (remove_unused_layers no)
   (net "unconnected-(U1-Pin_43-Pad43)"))
  (pad "44" thru_hole circle (at 25.4 53.34) (size 2 2) (drill 1) (layers "*.Cu" "*.Mask") (remove_unused_layers no)
   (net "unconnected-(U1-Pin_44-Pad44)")))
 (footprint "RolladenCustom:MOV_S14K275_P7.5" (layer "F.Cu") (at 52 27)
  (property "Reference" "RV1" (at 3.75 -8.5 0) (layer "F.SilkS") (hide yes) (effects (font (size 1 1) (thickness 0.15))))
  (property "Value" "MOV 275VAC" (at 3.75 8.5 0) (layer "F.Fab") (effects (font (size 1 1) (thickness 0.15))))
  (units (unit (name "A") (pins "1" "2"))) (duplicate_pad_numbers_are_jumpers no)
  (pad "1" thru_hole rect (at 0 0) (size 2.4 2.4) (drill 1.2) (layers "*.Cu" "*.Mask") (remove_unused_layers no) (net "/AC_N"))
  (pad "2" thru_hole circle (at 7.5 0) (size 2.4 2.4) (drill 1.2) (layers "*.Cu" "*.Mask") (remove_unused_layers no) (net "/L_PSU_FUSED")))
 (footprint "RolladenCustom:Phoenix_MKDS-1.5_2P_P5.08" (layer "F.Cu") (at 131 45)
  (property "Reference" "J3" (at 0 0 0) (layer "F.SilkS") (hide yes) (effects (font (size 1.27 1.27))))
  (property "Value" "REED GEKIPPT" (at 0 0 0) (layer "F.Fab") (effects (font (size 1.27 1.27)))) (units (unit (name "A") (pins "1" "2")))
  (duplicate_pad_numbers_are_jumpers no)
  (pad "1" thru_hole rect (at 0 0) (size 2.4 2.4) (drill 1.2) (layers "*.Cu" "*.Mask") (remove_unused_layers no) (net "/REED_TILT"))
  (pad "2" thru_hole circle (at 5.08 0) (size 2.4 2.4) (drill 1.2) (layers "*.Cu" "*.Mask") (remove_unused_layers no) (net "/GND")))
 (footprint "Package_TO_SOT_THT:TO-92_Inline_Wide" (layer "F.Cu") (at 150 58)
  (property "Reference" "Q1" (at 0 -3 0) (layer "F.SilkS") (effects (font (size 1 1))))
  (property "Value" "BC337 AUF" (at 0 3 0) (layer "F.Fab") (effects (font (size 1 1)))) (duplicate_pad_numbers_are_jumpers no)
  (pad "1" thru_hole circle (at -2.54 0) (size 1.8 1.8) (drill 0.9) (layers "*.Cu" "*.Mask") (remove_unused_layers no) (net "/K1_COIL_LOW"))
  (pad "2" thru_hole circle (at 0 0) (size 1.8 1.8) (drill 0.9) (layers "*.Cu" "*.Mask") (remove_unused_layers no) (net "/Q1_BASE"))
  (pad "3" thru_hole circle (at 2.54 0) (size 1.8 1.8) (drill 0.9) (layers "*.Cu" "*.Mask") (remove_unused_layers no) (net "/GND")))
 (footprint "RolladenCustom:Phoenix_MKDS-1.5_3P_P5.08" (layer "F.Cu") (at 23 25)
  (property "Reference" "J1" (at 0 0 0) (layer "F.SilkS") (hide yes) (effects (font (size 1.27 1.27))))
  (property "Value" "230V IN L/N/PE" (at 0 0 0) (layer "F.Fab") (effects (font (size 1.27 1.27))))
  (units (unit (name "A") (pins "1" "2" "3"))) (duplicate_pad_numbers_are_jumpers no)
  (pad "1" thru_hole rect (at 0 0) (size 2.4 2.4) (drill 1.2) (layers "*.Cu" "*.Mask") (remove_unused_layers no) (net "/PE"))
  (pad "2" thru_hole circle (at 5.08 0) (size 2.4 2.4) (drill 1.2) (layers "*.Cu" "*.Mask") (remove_unused_layers no) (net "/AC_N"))
  (pad "3" thru_hole circle (at 10.16 0) (size 2.4 2.4) (drill 1.2) (layers "*.Cu" "*.Mask") (remove_unused_layers no) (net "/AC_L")))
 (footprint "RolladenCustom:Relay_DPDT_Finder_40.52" (layer "F.Cu") (at 88 94 180)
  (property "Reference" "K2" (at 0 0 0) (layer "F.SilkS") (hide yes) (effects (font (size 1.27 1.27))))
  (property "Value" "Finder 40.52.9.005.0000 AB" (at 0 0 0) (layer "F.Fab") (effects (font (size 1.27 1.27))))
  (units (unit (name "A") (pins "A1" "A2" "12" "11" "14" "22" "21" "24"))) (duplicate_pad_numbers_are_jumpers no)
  (pad "11" thru_hole circle (at 20.32 0) (size 2.4 2.4) (drill 1.2) (layers "*.Cu" "*.Mask") (remove_unused_layers no) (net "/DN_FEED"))
  (pad "12" thru_hole circle (at 15.32 0) (size 2.4 2.4) (drill 1.2) (layers "*.Cu" "*.Mask") (remove_unused_layers no)
   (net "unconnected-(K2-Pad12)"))
  (pad "14" thru_hole circle (at 25.32 0) (size 2.4 2.4) (drill 1.2) (layers "*.Cu" "*.Mask") (remove_unused_layers no) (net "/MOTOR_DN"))
  (pad "21" thru_hole circle (at 20.32 7.62) (size 2.4 2.4) (drill 1.2) (layers "*.Cu" "*.Mask") (remove_unused_layers no) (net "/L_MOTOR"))
  (pad "22" thru_hole circle (at 15.32 7.62) (size 2.4 2.4) (drill 1.2) (layers "*.Cu" "*.Mask") (remove_unused_layers no) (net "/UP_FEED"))
  (pad "24" thru_hole circle (at 25.32 7.62) (size 2.4 2.4) (drill 1.2) (layers "*.Cu" "*.Mask") (remove_unused_layers no)
   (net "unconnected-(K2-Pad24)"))
  (pad "A1" thru_hole circle (at 0 0) (size 2.4 2.4) (drill 1.2) (layers "*.Cu" "*.Mask") (remove_unused_layers no) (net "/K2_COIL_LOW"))
  (pad "A2" thru_hole circle (at 0 7.62) (size 2.4 2.4) (drill 1.2) (layers "*.Cu" "*.Mask") (remove_unused_layers no) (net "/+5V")))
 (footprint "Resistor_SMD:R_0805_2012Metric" (layer "F.Cu") (at 143 64)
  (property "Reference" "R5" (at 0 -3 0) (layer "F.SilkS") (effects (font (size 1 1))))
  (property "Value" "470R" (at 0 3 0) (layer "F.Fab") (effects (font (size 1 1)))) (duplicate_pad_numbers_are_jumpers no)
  (pad "1" smd roundrect (at -1 0) (size 1.2 1.4) (layers "F.Cu" "F.Mask" "F.Paste") (roundrect_rratio 0.25) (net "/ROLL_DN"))
  (pad "2" smd roundrect (at 1 0) (size 1.2 1.4) (layers "F.Cu" "F.Mask" "F.Paste") (roundrect_rratio 0.25) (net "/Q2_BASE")))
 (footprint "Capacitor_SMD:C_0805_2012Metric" (layer "F.Cu") (at 149 28)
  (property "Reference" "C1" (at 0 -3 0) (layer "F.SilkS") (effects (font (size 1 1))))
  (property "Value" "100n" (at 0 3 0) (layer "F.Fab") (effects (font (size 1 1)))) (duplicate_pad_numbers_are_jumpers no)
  (pad "1" smd roundrect (at -1 0) (size 1.2 1.4) (layers "F.Cu" "F.Mask" "F.Paste") (roundrect_rratio 0.25) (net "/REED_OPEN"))
  (pad "2" smd roundrect (at 1 0) (size 1.2 1.4) (layers "F.Cu" "F.Mask" "F.Paste") (roundrect_rratio 0.25) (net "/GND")))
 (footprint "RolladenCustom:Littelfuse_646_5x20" (layer "F.Cu") (at 28 79.8 90)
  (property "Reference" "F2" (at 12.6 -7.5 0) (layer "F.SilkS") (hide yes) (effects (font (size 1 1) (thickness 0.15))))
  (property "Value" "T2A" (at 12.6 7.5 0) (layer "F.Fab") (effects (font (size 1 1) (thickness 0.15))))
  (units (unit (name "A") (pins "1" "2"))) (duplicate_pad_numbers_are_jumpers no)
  (pad "1" thru_hole rect (at 0 0) (size 2.4 2.4) (drill 1.4) (layers "*.Cu" "*.Mask") (remove_unused_layers no) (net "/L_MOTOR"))
  (pad "2" thru_hole circle (at 25.2 0) (size 2.4 2.4) (drill 1.4) (layers "*.Cu" "*.Mask") (remove_unused_layers no) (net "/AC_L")))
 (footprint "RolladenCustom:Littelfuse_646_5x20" (layer "F.Cu") (at 41 27)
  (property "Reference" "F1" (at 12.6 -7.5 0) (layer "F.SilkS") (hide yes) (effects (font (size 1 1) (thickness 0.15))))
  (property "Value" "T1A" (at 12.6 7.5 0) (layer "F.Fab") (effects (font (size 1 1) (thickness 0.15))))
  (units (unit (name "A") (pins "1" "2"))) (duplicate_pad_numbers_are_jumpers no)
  (pad "1" thru_hole rect (at 0 0) (size 2.4 2.4) (drill 1.4) (layers "*.Cu" "*.Mask") (remove_unused_layers no) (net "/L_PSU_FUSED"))
  (pad "2" thru_hole circle (at 25.2 0) (size 2.4 2.4) (drill 1.4) (layers "*.Cu" "*.Mask") (remove_unused_layers no) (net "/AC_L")))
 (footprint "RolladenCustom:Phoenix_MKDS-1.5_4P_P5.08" (layer "F.Cu") (at 112 90)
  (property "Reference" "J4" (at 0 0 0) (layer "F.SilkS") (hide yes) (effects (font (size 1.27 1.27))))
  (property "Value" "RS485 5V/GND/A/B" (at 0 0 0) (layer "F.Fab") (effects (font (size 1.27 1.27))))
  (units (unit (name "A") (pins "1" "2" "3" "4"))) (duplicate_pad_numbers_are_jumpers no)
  (pad "1" thru_hole rect (at 0 0) (size 2.4 2.4) (drill 1.2) (layers "*.Cu" "*.Mask") (remove_unused_layers no) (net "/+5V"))
  (pad "2" thru_hole circle (at 5.08 0) (size 2.4 2.4) (drill 1.2) (layers "*.Cu" "*.Mask") (remove_unused_layers no) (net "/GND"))
  (pad "3" thru_hole circle (at 10.16 0) (size 2.4 2.4) (drill 1.2) (layers "*.Cu" "*.Mask") (remove_unused_layers no) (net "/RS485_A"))
  (pad "4" thru_hole circle (at 15.24 0) (size 2.4 2.4) (drill 1.2) (layers "*.Cu" "*.Mask") (remove_unused_layers no) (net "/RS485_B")))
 (gr_rect (start 20 20) (end 170 110) (stroke (width 0.5) (type default)) (fill no) (layer "Edge.Cuts"))
 (via (at 126 40) (size 0.8) (drill 0.4) (layers "F.Cu" "B.Cu") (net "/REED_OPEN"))
 (via (at 130 40) (size 0.8) (drill 0.4) (layers "F.Cu" "B.Cu") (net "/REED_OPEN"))
 (segment (start 130 32) (end 131 30) (width 0.3) (layer "F.Cu") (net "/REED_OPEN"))
 (segment (start 120 77.1) (end 120 24.5) (width 0.3) (layer "F.Cu") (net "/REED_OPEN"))
 (segment (start 120 24.5) (end 131 24.5) (width 0.3) (layer "F.Cu") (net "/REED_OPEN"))
 (segment (start 131 24.5) (end 131 30) (width 0.3) (layer "F.Cu") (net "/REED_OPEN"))
 (segment (start 131 30) (end 132 33) (width 0.3) (layer "B.Cu") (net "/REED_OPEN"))
 (segment (start 132 33) (end 146 33) (width 0.3) (layer "B.Cu") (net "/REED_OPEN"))
 (via (at 146 33) (size 0.8) (drill 0.4) (layers "F.Cu" "B.Cu") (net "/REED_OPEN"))
 (segment (start 146 33) (end 146 28) (width 0.3) (layer "F.Cu") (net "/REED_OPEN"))
 (segment (start 146 28) (end 144 28) (width 0.3) (layer "F.Cu") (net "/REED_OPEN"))
 (segment (start 146 28) (end 148 28) (width 0.3) (layer "F.Cu") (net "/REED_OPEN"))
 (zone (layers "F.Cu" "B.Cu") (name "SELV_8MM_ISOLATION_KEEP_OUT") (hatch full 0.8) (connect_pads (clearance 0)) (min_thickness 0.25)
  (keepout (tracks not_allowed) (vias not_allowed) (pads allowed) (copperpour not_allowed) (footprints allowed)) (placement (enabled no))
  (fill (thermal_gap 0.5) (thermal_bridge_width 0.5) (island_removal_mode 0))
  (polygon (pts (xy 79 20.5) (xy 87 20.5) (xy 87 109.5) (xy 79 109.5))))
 (segment (start 157.7 31) (end 154 31) (width 0.6) (layer "F.Cu") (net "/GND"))
 (segment (start 154 31) (end 154 23.5) (width 0.6) (layer "F.Cu") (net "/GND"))
 (segment (start 154 23.5) (end 138 23.5) (width 0.6) (layer "F.Cu") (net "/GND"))
 (segment (start 138 23.5) (end 138 26) (width 0.6) (layer "F.Cu") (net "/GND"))
 (segment (start 162.3 31) (end 164.5 32.5) (width 0.8) (layer "F.Cu") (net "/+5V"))
 (via (at 164.5 32.5) (size 1.4) (drill 0.7) (layers "F.Cu" "B.Cu") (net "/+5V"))
 (segment (start 164.5 32.5) (end 166 32.5) (width 0.8) (layer "B.Cu") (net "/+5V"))
 (segment (start 166 32.5) (end 166 21.2) (width 0.8) (layer "B.Cu") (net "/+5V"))
 (segment (start 166 21.2) (end 98 21.2) (width 0.8) (layer "B.Cu") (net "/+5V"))
 (segment (start 98 21.2) (end 98 28) (width 0.8) (layer "B.Cu") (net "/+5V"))
 (segment (start 160 25.4) (end 160 31) (width 0.5) (layer "F.Cu") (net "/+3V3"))
 (segment (start 160 25.4) (end 168 25.4) (width 0.5) (layer "F.Cu") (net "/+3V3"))
 (segment (start 168 25.4) (end 168 41) (width 0.5) (layer "F.Cu") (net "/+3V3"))
 (segment (start 168 41) (end 164 41) (width 0.5) (layer "F.Cu") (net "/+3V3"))
 (segment (start 164 41) (end 164 43.095) (width 0.5) (layer "F.Cu") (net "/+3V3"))
 (segment (start 164 43.095) (end 161.7 43.095) (width 0.5) (layer "F.Cu") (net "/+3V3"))
 (segment (start 161.7 46.905) (end 168 46.905) (width 0.6) (layer "F.Cu") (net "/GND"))
 (segment (start 168 46.905) (end 168 52) (width 0.6) (layer "F.Cu") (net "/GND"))
 (segment (start 168 52) (end 128 52) (width 0.6) (layer "F.Cu") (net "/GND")))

